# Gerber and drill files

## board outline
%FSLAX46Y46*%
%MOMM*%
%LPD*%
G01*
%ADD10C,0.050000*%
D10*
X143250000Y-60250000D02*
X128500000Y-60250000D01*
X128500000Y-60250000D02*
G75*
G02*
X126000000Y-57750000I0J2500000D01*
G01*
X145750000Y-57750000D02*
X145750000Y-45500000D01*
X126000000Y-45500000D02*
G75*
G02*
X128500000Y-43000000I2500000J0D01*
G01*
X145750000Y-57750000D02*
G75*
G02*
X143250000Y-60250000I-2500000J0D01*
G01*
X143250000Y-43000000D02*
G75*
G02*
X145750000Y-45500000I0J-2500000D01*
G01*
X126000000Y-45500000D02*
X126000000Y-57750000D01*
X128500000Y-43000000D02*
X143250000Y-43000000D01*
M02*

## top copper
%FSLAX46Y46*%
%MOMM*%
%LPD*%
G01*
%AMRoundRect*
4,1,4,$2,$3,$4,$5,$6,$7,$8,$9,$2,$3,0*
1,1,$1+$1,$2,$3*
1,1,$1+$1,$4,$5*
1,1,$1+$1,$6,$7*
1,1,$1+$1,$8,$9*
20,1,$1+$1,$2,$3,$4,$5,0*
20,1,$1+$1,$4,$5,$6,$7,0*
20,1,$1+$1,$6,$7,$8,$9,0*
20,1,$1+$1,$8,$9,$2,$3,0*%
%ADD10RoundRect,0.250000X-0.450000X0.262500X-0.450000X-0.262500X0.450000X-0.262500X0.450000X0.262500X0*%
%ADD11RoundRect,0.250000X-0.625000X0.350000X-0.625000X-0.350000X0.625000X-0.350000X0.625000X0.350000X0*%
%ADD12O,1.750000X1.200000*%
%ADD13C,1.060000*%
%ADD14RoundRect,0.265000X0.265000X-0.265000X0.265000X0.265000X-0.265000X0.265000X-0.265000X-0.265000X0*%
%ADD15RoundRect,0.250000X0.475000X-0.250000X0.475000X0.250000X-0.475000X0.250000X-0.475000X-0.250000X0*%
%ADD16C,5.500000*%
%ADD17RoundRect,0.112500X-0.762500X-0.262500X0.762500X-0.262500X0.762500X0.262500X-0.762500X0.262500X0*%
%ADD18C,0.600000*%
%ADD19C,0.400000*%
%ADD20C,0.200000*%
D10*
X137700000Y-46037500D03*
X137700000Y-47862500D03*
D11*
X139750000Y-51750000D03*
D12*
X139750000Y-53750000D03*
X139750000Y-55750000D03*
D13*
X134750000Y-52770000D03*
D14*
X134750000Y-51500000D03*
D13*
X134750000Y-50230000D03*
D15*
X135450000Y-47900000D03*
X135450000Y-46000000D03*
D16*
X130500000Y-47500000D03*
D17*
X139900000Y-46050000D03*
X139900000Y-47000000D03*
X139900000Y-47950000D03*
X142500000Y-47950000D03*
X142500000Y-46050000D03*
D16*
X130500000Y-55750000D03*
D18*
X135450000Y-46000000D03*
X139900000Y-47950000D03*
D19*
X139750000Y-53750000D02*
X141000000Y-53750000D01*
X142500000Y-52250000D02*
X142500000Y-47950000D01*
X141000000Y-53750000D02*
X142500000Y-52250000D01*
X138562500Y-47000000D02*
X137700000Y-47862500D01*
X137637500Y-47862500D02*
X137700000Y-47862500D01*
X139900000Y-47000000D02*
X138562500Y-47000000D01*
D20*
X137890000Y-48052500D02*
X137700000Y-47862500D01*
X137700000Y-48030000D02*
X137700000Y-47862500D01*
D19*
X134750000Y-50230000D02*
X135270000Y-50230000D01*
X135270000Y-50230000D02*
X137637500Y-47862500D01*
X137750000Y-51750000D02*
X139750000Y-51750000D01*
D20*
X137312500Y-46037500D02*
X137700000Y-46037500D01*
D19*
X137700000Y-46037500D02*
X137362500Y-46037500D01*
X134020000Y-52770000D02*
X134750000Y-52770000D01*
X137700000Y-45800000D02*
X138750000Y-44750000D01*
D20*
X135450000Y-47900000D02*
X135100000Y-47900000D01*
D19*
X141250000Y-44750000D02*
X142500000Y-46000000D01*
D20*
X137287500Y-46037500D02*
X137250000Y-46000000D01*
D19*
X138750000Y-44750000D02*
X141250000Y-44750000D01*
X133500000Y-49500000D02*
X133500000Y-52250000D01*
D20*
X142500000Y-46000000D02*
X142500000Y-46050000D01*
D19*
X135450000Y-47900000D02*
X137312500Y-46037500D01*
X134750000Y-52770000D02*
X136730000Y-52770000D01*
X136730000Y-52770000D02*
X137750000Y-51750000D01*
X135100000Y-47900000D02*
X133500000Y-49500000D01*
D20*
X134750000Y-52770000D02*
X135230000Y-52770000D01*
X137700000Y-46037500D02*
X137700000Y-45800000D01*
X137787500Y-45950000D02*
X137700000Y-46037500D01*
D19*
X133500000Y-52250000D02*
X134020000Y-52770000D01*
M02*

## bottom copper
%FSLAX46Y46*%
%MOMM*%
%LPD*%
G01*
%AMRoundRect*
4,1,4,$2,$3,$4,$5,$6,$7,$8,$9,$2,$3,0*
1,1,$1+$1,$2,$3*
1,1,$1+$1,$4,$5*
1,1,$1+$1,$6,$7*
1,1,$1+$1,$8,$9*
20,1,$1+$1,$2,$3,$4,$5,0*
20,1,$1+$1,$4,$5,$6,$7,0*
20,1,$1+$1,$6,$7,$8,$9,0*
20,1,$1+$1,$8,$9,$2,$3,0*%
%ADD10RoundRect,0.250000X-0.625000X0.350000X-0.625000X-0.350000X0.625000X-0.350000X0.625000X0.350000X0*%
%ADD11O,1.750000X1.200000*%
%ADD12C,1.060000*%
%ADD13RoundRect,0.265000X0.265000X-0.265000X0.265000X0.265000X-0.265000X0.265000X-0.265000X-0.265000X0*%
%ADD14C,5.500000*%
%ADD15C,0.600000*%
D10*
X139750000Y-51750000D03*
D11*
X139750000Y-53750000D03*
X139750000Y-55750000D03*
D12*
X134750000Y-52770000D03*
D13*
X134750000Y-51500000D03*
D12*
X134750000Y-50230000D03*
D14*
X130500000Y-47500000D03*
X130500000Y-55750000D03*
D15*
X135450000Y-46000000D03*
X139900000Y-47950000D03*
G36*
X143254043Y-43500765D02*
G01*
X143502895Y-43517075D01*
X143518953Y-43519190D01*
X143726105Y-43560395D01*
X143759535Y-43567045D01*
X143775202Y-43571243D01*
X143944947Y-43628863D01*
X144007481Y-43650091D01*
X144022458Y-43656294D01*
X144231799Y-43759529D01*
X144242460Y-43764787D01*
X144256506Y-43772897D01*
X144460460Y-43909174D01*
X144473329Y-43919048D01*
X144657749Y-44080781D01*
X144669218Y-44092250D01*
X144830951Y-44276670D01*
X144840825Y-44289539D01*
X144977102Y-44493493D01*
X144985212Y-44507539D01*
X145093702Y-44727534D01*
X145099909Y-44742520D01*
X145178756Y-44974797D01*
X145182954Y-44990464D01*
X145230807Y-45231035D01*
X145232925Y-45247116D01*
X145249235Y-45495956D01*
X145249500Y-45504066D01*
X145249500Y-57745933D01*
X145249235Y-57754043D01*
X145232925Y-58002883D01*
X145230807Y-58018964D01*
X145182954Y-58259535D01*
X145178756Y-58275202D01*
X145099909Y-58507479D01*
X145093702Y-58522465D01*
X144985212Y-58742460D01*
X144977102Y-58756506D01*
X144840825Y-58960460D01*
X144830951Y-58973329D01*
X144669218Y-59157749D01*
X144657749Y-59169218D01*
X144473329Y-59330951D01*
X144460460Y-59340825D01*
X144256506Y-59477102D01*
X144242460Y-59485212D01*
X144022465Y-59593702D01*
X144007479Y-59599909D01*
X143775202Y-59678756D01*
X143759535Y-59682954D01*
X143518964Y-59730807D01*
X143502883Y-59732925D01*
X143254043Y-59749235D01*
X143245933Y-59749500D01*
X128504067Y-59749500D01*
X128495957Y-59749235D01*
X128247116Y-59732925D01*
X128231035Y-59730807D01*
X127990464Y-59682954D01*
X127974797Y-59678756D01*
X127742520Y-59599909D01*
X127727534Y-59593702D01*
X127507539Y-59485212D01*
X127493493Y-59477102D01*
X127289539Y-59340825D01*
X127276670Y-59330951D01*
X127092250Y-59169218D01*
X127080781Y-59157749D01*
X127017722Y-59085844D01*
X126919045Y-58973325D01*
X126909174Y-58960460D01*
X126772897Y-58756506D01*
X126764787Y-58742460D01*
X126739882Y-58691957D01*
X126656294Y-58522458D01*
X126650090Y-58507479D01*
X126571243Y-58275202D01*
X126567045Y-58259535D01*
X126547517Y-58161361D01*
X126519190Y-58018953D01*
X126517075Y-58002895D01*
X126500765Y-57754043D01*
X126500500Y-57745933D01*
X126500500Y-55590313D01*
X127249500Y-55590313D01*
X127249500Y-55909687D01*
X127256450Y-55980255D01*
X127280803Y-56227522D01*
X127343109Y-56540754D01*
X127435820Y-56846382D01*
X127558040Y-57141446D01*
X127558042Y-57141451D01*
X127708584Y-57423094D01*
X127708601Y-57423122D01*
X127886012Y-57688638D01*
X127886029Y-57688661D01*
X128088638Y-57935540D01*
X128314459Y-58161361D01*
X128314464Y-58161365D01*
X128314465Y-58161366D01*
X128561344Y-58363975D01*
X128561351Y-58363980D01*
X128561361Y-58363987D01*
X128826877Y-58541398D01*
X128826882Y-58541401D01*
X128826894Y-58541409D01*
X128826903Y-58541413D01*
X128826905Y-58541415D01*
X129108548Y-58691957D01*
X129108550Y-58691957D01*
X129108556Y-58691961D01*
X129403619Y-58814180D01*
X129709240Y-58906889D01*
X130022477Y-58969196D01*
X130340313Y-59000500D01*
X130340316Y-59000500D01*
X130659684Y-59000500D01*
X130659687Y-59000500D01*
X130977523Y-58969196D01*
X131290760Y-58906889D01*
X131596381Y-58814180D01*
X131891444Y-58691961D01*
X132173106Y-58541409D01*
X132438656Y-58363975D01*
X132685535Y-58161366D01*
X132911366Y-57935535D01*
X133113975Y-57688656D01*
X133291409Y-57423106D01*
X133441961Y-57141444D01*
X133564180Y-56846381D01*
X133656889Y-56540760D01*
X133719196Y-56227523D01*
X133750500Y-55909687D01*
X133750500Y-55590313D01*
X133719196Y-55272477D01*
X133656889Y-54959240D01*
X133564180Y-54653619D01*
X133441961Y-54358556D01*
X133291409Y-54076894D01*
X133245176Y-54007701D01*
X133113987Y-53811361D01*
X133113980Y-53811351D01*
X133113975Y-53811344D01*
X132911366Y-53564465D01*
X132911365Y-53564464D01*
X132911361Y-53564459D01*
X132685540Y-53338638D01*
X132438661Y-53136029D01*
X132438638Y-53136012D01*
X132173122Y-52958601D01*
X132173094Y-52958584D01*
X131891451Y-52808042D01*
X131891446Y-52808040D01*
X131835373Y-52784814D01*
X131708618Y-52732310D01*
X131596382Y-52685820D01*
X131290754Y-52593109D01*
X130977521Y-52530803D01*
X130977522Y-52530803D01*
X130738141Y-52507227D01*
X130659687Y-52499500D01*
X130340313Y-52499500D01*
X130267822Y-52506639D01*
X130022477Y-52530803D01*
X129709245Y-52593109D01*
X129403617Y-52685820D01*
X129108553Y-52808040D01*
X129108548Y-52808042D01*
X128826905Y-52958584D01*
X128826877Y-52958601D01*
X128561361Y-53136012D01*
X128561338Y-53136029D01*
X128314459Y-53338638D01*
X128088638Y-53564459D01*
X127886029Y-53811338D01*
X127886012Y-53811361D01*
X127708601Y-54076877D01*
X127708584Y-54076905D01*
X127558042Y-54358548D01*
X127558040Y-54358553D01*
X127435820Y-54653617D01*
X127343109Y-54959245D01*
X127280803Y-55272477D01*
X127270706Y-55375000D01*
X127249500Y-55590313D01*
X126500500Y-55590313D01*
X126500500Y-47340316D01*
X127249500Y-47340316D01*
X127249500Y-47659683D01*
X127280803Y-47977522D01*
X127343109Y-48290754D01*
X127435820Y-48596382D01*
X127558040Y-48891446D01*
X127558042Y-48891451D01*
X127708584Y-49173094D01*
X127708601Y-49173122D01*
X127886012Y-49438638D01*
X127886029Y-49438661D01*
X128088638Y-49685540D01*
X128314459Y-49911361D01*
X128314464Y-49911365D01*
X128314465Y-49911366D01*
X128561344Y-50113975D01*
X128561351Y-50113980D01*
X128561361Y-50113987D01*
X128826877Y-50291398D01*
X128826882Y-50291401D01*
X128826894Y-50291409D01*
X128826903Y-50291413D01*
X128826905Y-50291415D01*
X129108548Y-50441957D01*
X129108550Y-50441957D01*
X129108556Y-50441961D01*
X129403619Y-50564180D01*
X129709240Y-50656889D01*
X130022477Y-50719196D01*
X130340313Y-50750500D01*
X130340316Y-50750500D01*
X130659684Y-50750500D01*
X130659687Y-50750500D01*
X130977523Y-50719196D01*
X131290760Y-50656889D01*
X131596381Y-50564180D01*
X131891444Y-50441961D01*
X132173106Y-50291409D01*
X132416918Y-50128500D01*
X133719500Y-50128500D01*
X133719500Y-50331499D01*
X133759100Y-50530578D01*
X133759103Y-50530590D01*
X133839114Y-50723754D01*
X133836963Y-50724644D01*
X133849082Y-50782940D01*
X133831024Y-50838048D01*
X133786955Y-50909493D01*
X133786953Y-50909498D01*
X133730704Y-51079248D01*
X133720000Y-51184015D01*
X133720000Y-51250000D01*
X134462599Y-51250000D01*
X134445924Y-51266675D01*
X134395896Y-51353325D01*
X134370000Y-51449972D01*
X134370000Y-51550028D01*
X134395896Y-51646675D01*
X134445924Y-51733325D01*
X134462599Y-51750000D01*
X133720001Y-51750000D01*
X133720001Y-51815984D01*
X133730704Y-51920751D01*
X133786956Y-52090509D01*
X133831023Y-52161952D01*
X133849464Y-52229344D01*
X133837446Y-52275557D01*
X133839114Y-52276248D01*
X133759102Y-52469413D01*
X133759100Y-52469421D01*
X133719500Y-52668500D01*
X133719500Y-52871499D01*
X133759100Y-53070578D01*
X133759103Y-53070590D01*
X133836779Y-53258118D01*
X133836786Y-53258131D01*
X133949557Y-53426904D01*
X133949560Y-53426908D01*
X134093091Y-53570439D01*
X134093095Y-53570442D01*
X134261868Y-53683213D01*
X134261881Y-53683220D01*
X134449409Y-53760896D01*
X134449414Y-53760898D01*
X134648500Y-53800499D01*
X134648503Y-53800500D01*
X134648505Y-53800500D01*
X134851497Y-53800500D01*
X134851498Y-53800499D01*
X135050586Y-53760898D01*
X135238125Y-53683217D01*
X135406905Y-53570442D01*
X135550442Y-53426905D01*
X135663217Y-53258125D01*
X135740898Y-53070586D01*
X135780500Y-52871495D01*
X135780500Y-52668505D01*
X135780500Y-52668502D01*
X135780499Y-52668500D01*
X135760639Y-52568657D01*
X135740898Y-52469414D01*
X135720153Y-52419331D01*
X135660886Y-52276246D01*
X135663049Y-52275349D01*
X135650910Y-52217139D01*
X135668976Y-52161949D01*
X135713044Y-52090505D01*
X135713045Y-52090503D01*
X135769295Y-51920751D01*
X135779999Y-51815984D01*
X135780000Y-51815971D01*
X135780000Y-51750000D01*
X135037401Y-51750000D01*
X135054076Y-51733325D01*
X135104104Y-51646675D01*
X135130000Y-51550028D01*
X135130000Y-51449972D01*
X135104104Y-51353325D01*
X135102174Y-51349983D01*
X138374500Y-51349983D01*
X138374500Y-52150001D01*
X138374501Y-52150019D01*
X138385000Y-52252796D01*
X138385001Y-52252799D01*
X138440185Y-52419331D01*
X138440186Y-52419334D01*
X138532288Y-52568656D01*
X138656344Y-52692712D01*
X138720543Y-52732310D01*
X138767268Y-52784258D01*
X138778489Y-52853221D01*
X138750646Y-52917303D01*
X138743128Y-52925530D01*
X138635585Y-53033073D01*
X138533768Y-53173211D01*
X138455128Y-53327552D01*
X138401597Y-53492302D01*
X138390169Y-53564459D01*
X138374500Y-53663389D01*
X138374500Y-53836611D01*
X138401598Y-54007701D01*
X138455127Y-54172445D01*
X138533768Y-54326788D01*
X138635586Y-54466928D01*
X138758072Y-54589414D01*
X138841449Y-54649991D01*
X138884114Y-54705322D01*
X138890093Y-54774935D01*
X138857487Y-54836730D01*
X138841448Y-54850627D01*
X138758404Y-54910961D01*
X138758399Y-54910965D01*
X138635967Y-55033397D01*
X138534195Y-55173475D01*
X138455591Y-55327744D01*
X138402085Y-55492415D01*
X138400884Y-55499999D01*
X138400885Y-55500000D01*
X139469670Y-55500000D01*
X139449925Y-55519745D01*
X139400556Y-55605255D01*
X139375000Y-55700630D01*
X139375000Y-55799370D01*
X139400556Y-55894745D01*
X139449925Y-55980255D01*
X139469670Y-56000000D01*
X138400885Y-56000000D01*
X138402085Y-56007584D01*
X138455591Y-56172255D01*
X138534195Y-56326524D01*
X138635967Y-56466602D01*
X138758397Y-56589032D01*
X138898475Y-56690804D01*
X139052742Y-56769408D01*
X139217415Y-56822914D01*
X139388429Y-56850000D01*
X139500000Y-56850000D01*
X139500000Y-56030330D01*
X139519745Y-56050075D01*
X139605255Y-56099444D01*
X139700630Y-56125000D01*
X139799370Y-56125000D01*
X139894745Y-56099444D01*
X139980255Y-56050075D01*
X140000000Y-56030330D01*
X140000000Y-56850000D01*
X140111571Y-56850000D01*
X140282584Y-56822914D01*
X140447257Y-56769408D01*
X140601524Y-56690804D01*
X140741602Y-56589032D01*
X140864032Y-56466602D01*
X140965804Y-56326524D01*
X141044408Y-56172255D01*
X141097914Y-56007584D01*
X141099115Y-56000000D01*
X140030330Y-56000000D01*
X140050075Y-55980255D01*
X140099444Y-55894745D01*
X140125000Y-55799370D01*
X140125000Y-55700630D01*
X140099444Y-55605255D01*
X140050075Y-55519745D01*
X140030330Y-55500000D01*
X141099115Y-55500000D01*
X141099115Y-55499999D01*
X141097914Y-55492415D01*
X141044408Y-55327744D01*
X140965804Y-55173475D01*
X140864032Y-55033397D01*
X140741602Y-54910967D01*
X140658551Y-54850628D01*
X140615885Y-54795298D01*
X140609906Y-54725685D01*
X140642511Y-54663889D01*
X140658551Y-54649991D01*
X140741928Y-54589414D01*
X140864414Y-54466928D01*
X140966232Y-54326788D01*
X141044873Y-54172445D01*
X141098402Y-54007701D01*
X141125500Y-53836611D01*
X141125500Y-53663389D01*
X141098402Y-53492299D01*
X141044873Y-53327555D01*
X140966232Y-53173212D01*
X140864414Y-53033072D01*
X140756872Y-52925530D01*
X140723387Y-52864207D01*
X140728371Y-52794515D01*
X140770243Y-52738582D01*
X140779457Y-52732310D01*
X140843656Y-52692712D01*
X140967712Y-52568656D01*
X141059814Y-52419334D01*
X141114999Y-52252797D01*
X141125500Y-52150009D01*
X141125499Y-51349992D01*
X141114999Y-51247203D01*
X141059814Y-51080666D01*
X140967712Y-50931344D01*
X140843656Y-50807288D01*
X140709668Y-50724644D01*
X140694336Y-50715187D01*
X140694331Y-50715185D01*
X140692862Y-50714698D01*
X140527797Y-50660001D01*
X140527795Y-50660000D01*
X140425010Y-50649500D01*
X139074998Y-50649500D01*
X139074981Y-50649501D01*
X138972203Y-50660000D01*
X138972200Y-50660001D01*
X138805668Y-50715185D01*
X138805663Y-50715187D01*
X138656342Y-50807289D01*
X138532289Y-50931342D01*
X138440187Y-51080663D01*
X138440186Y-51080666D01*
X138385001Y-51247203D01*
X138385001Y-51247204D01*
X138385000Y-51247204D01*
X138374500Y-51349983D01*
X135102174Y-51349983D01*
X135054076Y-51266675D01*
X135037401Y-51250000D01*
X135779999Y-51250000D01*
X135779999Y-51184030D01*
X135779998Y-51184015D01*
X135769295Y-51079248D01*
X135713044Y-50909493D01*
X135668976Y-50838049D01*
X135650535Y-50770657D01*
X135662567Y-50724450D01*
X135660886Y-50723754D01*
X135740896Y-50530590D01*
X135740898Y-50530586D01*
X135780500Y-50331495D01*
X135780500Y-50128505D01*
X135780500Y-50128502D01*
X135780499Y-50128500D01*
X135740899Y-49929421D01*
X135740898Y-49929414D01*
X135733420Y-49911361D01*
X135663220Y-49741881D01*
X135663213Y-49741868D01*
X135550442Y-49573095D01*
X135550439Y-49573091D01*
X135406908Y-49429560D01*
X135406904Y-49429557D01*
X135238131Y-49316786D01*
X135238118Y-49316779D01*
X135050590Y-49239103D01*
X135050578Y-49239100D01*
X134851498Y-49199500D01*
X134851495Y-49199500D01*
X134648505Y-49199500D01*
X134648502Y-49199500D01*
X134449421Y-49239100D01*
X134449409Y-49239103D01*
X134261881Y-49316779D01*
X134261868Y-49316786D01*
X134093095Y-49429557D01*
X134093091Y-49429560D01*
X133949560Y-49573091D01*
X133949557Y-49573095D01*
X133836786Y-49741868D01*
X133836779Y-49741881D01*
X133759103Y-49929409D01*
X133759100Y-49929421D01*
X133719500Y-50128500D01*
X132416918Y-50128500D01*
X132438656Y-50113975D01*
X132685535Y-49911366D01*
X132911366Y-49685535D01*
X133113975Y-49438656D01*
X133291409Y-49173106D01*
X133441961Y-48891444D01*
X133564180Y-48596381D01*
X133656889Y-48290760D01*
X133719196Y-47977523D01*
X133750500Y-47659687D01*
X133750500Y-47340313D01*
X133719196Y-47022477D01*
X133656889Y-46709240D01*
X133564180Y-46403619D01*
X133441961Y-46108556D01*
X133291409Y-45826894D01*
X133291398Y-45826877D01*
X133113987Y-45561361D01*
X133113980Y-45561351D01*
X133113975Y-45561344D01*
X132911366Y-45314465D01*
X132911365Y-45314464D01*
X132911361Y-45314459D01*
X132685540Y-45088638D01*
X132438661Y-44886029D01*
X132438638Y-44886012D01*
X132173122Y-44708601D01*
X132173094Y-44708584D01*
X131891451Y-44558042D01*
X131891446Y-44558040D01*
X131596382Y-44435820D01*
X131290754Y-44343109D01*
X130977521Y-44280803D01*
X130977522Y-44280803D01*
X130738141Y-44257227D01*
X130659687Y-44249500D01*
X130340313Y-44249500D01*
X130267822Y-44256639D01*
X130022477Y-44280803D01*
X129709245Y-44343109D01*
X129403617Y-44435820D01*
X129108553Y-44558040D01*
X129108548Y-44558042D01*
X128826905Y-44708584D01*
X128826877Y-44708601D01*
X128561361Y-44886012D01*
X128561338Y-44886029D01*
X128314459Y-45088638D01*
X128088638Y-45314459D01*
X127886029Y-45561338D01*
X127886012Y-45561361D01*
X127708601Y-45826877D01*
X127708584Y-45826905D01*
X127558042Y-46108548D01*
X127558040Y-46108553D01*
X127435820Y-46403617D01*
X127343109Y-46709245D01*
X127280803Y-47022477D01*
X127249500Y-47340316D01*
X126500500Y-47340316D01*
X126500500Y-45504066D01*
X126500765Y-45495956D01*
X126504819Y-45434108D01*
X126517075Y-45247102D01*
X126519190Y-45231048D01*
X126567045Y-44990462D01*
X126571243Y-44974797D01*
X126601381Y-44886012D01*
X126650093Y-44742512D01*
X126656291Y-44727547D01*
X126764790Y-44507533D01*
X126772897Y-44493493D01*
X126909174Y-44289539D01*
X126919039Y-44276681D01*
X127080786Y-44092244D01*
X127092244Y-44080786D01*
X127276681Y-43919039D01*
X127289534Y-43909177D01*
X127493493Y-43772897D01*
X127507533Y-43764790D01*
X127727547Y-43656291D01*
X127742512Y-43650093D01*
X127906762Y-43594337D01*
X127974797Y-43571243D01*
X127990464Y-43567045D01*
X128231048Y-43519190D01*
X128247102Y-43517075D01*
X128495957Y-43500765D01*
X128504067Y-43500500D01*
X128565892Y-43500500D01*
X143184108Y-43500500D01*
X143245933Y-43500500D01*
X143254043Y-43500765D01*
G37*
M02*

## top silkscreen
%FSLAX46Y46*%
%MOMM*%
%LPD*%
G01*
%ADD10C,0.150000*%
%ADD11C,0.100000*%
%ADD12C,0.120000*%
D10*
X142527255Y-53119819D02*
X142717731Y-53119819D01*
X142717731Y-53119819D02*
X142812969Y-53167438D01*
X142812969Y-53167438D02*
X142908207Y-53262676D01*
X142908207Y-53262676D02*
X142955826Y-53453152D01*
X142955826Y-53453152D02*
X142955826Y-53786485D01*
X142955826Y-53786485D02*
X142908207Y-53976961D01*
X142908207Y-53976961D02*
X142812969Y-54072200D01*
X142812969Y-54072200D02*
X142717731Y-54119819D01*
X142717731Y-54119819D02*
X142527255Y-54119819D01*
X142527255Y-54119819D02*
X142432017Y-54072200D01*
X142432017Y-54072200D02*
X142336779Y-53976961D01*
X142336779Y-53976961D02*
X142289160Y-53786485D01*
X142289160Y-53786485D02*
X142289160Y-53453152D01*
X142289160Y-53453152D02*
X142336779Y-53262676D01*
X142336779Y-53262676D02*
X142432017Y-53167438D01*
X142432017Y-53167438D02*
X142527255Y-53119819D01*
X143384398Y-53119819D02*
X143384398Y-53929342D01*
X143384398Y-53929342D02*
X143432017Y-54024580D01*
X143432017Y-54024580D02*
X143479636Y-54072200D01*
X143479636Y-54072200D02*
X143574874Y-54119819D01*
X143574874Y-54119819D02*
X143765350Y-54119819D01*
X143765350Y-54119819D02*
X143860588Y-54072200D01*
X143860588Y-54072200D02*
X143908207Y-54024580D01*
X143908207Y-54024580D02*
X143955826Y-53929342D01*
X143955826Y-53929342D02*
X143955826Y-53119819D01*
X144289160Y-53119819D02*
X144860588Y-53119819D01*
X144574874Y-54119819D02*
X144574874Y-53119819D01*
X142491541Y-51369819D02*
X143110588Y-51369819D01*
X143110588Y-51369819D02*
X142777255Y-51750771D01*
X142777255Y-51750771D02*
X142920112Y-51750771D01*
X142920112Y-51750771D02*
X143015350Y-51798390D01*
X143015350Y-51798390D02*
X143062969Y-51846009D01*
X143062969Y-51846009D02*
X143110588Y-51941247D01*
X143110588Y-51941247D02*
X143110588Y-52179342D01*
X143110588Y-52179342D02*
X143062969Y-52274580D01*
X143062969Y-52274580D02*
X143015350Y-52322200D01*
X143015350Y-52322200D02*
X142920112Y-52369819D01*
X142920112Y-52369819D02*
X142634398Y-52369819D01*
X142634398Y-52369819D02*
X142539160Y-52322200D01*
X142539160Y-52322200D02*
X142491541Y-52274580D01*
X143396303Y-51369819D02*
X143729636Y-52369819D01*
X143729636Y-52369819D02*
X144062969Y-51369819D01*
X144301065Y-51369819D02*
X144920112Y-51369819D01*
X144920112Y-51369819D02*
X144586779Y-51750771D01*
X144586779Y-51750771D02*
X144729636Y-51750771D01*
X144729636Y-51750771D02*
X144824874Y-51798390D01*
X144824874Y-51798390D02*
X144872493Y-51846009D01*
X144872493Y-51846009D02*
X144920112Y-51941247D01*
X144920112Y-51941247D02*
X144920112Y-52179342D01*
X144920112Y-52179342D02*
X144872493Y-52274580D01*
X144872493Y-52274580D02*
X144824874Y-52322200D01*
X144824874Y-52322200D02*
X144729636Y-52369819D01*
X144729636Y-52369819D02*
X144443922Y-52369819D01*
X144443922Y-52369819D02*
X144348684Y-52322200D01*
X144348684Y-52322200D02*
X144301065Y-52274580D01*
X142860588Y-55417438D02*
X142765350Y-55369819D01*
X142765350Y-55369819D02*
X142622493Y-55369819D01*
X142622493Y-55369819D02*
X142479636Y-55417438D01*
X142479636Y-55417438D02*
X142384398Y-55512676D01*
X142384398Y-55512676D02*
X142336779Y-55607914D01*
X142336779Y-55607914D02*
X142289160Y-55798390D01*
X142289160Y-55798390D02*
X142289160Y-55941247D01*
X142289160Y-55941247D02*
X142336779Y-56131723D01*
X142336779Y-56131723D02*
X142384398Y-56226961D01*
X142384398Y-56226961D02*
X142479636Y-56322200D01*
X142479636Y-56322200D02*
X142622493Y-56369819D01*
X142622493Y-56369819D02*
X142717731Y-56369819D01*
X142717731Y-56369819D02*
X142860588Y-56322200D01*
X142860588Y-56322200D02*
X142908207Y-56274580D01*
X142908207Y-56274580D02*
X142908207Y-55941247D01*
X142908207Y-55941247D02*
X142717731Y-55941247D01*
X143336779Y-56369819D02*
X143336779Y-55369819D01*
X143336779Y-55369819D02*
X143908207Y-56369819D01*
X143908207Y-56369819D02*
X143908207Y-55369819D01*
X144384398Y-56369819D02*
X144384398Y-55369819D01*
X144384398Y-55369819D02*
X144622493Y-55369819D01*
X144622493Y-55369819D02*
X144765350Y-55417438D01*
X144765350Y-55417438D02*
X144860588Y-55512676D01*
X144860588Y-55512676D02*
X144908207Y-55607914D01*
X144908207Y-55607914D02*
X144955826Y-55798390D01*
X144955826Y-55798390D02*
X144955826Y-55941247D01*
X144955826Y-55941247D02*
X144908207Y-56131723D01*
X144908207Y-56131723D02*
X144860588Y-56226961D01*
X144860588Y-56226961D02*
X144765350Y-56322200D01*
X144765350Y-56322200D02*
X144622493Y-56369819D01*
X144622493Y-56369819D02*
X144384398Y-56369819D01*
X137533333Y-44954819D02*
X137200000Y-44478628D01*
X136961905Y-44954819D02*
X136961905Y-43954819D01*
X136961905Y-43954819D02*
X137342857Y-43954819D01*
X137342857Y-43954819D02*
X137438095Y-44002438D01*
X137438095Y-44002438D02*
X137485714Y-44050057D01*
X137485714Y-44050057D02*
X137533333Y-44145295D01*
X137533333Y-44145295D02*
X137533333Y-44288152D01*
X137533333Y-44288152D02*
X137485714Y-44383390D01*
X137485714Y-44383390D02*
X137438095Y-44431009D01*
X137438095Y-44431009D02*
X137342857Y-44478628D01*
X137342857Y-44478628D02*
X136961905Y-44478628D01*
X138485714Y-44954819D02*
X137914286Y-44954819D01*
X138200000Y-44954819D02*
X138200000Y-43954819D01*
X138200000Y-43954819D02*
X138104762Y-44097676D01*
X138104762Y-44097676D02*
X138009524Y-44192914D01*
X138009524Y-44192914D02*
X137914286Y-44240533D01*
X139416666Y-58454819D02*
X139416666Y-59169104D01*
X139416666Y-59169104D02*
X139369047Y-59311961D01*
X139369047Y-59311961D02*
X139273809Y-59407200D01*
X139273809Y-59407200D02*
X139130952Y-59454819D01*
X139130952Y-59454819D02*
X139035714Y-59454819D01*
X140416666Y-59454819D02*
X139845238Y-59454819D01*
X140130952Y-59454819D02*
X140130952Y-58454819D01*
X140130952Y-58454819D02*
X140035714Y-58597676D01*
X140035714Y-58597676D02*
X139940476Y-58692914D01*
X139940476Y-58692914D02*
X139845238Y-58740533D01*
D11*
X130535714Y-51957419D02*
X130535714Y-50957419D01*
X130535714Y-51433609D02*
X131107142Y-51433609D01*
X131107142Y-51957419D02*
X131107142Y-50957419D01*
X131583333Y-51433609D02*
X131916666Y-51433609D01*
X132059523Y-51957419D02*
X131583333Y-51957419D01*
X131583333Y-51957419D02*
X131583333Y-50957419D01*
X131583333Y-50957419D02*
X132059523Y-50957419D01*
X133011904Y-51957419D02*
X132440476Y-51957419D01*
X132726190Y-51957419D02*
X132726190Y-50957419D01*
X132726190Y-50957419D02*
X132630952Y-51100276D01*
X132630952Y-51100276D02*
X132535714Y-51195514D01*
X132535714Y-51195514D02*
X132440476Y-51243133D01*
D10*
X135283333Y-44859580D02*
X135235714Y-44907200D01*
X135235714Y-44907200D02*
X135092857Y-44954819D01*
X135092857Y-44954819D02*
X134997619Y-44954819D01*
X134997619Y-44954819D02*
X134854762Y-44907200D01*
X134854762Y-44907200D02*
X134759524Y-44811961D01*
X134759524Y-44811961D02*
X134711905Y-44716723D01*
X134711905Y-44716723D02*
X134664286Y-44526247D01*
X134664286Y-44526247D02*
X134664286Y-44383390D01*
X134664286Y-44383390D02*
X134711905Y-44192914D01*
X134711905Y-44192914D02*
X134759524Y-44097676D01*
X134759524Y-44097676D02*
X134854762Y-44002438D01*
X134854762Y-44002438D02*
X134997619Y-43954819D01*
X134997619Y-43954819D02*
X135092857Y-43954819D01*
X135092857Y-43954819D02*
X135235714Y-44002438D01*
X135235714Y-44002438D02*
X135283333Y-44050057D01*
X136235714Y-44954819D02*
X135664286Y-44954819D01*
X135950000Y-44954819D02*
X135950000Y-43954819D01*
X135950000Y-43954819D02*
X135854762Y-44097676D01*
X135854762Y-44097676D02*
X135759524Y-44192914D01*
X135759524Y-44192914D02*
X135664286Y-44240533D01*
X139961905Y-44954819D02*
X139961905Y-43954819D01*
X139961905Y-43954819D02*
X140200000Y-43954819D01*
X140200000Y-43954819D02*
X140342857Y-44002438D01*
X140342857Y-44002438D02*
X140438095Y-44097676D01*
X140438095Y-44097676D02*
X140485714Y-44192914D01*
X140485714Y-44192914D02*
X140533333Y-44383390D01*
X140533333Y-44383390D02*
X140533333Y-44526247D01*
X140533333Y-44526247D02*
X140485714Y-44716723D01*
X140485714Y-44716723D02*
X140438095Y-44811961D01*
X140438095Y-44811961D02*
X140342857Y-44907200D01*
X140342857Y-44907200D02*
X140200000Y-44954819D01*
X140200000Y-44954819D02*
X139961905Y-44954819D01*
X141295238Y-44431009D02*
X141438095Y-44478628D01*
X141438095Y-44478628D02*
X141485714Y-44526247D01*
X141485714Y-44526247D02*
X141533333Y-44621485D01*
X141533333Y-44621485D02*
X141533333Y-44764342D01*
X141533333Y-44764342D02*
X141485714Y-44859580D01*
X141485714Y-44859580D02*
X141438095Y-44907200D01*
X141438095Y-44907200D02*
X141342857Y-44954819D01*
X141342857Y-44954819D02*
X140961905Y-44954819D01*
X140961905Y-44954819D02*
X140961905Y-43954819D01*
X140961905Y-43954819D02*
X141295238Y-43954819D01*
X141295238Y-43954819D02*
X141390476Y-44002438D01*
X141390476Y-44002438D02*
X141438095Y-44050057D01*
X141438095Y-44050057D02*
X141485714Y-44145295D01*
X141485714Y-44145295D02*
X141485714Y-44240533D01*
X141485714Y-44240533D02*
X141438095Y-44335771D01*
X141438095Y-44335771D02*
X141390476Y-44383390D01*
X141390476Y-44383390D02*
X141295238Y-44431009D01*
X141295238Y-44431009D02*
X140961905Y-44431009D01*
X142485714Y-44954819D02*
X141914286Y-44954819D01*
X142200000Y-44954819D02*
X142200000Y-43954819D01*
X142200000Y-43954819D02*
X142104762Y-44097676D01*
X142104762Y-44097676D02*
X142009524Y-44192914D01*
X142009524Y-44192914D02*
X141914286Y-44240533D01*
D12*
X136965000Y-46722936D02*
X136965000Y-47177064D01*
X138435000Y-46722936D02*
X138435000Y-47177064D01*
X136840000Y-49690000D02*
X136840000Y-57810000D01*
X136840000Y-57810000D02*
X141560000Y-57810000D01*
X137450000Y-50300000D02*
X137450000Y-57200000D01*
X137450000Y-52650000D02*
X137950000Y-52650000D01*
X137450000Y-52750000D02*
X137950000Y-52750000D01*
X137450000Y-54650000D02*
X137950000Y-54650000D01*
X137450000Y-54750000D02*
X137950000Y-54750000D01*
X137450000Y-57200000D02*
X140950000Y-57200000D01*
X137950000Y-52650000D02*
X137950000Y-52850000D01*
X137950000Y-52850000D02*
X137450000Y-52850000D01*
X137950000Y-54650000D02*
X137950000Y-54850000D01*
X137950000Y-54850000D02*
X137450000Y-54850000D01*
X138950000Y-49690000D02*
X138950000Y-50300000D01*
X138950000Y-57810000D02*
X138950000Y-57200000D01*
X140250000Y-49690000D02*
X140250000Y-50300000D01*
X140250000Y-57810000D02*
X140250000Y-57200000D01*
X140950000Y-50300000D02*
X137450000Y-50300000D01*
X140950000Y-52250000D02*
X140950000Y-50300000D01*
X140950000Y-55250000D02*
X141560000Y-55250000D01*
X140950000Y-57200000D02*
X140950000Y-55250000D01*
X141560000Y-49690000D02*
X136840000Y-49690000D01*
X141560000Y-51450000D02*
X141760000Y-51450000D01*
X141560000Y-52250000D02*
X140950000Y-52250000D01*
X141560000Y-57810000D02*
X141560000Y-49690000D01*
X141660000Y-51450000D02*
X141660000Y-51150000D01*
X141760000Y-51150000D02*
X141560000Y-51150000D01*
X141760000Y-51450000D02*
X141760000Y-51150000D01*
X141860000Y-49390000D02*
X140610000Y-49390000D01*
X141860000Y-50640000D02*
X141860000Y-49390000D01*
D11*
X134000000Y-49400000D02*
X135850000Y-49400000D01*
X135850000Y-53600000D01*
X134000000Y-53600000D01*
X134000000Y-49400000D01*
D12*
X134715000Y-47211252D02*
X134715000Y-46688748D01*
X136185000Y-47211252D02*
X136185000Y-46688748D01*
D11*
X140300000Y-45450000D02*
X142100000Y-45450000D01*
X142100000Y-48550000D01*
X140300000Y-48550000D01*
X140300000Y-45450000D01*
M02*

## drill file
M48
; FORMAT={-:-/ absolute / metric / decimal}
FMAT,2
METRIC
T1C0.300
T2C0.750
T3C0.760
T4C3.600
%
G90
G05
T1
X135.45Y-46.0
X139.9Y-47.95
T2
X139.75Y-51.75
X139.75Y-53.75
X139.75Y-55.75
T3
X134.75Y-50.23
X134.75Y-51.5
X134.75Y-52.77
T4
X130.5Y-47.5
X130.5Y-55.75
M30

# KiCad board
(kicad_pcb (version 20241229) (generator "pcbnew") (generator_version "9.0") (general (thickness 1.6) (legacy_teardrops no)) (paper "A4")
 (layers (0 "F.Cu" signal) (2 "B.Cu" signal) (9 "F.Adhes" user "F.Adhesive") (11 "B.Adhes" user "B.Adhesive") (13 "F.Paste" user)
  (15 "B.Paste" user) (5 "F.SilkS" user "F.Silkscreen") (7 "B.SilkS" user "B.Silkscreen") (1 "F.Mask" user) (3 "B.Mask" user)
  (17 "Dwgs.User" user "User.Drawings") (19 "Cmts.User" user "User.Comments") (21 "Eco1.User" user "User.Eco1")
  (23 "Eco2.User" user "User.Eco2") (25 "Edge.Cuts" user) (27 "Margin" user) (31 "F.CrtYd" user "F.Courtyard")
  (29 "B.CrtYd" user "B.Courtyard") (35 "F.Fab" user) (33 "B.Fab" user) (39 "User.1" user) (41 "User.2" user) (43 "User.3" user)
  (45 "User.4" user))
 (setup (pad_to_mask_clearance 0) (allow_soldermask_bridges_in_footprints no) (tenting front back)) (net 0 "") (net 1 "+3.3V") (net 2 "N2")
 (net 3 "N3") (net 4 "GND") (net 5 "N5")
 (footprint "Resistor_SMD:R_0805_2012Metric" (layer "F.Cu") (at 137.7 46.95 -90)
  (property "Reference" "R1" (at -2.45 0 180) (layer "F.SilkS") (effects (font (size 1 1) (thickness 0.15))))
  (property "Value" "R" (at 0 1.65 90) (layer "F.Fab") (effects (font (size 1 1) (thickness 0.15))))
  (fp_line (start -0.227064 0.735) (end 0.227064 0.735) (stroke (width 0.12) (type solid)) (layer "F.SilkS"))
  (fp_line (start -0.227064 -0.735) (end 0.227064 -0.735) (stroke (width 0.12) (type solid)) (layer "F.SilkS"))
  (pad "1" smd roundrect (at -0.9125 0 270) (size 1.025 1.4) (layers "F.Cu" "F.Mask" "F.Paste") (roundrect_rratio 0.243902) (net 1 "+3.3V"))
  (pad "2" smd roundrect (at 0.9125 0 270) (size 1.025 1.4) (layers "F.Cu" "F.Mask" "F.Paste") (roundrect_rratio 0.243902) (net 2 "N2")))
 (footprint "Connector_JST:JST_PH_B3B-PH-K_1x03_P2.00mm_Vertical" (layer "F.Cu") (at 139.75 51.75 -90)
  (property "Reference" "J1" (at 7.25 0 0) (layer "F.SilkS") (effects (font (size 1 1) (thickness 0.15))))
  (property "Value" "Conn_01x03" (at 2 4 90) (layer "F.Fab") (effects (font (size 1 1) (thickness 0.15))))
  (fp_line (start -2.06 2.91) (end 6.06 2.91) (stroke (width 0.12) (type solid)) (layer "F.SilkS"))
  (fp_line (start 6.06 2.91) (end 6.06 -1.81) (stroke (width 0.12) (type solid)) (layer "F.SilkS"))
  (fp_line (start -1.45 2.3) (end 5.45 2.3) (stroke (width 0.12) (type solid)) (layer "F.SilkS"))
  (fp_line (start 0.9 2.3) (end 0.9 1.8) (stroke (width 0.12) (type solid)) (layer "F.SilkS"))
  (fp_line (start 1 2.3) (end 1 1.8) (stroke (width 0.12) (type solid)) (layer "F.SilkS"))
  (fp_line (start 2.9 2.3) (end 2.9 1.8) (stroke (width 0.12) (type solid)) (layer "F.SilkS"))
  (fp_line (start 3 2.3) (end 3 1.8) (stroke (width 0.12) (type solid)) (layer "F.SilkS"))
  (fp_line (start 5.45 2.3) (end 5.45 -1.2) (stroke (width 0.12) (type solid)) (layer "F.SilkS"))
  (fp_line (start 0.9 1.8) (end 1.1 1.8) (stroke (width 0.12) (type solid)) (layer "F.SilkS"))
  (fp_line (start 1.1 1.8) (end 1.1 2.3) (stroke (width 0.12) (type solid)) (layer "F.SilkS"))
  (fp_line (start 2.9 1.8) (end 3.1 1.8) (stroke (width 0.12) (type solid)) (layer "F.SilkS"))
  (fp_line (start 3.1 1.8) (end 3.1 2.3) (stroke (width 0.12) (type solid)) (layer "F.SilkS"))
  (fp_line (start -2.06 0.8) (end -1.45 0.8) (stroke (width 0.12) (type solid)) (layer "F.SilkS"))
  (fp_line (start 6.06 0.8) (end 5.45 0.8) (stroke (width 0.12) (type solid)) (layer "F.SilkS"))
  (fp_line (start -2.06 -0.5) (end -1.45 -0.5) (stroke (width 0.12) (type solid)) (layer "F.SilkS"))
  (fp_line (start 6.06 -0.5) (end 5.45 -0.5) (stroke (width 0.12) (type solid)) (layer "F.SilkS"))
  (fp_line (start -1.45 -1.2) (end -1.45 2.3) (stroke (width 0.12) (type solid)) (layer "F.SilkS"))
  (fp_line (start 0.5 -1.2) (end -1.45 -1.2) (stroke (width 0.12) (type solid)) (layer "F.SilkS"))
  (fp_line (start 3.5 -1.2) (end 3.5 -1.81) (stroke (width 0.12) (type solid)) (layer "F.SilkS"))
  (fp_line (start 5.45 -1.2) (end 3.5 -1.2) (stroke (width 0.12) (type solid)) (layer "F.SilkS"))
  (fp_line (start -2.06 -1.81) (end -2.06 2.91) (stroke (width 0.12) (type solid)) (layer "F.SilkS"))
  (fp_line (start -0.3 -1.81) (end -0.3 -2.01) (stroke (width 0.12) (type solid)) (layer "F.SilkS"))
  (fp_line (start 0.5 -1.81) (end 0.5 -1.2) (stroke (width 0.12) (type solid)) (layer "F.SilkS"))
  (fp_line (start 6.06 -1.81) (end -2.06 -1.81) (stroke (width 0.12) (type solid)) (layer "F.SilkS"))
  (fp_line (start -0.3 -1.91) (end -0.6 -1.91) (stroke (width 0.12) (type solid)) (layer "F.SilkS"))
  (fp_line (start -0.6 -2.01) (end -0.6 -1.81) (stroke (width 0.12) (type solid)) (layer "F.SilkS"))
  (fp_line (start -0.3 -2.01) (end -0.6 -2.01) (stroke (width 0.12) (type solid)) (layer "F.SilkS"))
  (fp_line (start -2.36 -2.11) (end -2.36 -0.86) (stroke (width 0.12) (type solid)) (layer "F.SilkS"))
  (fp_line (start -1.11 -2.11) (end -2.36 -2.11) (stroke (width 0.12) (type solid)) (layer "F.SilkS"))
  (pad "1" thru_hole roundrect (at 0 0 270) (size 1.2 1.75) (drill 0.75) (layers "*.Cu" "*.Mask") (remove_unused_layers no)
   (roundrect_rratio 0.208333) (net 1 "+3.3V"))
  (pad "2" thru_hole oval (at 2 0 270) (size 1.2 1.75) (drill 0.75) (layers "*.Cu" "*.Mask") (remove_unused_layers no) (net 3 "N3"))
  (pad "3" thru_hole oval (at 4 0 270) (size 1.2 1.75) (drill 0.75) (layers "*.Cu" "*.Mask") (remove_unused_layers no) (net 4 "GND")))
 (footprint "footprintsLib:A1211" (layer "F.Cu") (at 134.75 51.5 90)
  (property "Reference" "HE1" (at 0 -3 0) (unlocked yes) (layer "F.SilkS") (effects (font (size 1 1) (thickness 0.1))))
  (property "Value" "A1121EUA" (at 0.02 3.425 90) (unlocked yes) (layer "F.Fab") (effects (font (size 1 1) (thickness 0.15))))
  (fp_rect (start -2.1 -0.75) (end 2.1 1.1) (stroke (width 0.1) (type solid)) (fill no) (layer "F.SilkS"))
  (pad "1" thru_hole circle (at -1.27 0 90) (size 1.06 1.06) (drill 0.76) (layers "*.Cu" "*.Mask") (remove_unused_layers no) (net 1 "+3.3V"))
  (pad "2" thru_hole roundrect (at 0 0 90) (size 1.06 1.06) (drill 0.76) (layers "*.Cu" "*.Mask") (remove_unused_layers no)
   (roundrect_rratio 0.25) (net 4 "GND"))
  (pad "3" thru_hole circle (at 1.27 0 90) (size 1.06 1.06) (drill 0.76) (layers "*.Cu" "*.Mask") (remove_unused_layers no) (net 2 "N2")))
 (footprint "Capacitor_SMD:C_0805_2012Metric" (layer "F.Cu") (at 135.45 46.95 90)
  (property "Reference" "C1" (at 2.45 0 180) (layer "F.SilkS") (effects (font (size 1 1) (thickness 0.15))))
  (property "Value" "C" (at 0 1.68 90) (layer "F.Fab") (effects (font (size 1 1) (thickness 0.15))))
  (fp_line (start -0.261252 -0.735) (end 0.261252 -0.735) (stroke (width 0.12) (type solid)) (layer "F.SilkS"))
  (fp_line (start -0.261252 0.735) (end 0.261252 0.735) (stroke (width 0.12) (type solid)) (layer "F.SilkS"))
  (pad "1" smd roundrect (at -0.95 0 90) (size 1 1.45) (layers "F.Cu" "F.Mask" "F.Paste") (roundrect_rratio 0.25) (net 1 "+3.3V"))
  (pad "2" smd roundrect (at 0.95 0 90) (size 1 1.45) (layers "F.Cu" "F.Mask" "F.Paste") (roundrect_rratio 0.25) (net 4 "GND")))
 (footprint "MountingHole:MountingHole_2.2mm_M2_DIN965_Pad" (layer "F.Cu") (at 130.5 47.5)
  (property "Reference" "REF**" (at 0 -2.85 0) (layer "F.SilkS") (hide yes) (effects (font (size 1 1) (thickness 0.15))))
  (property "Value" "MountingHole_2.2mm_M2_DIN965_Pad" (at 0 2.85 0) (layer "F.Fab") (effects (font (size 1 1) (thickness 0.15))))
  (pad "1" thru_hole circle (at 0 0) (size 5.5 5.5) (drill 3.6) (layers "*.Cu" "*.Mask") (remove_unused_layers no) (zone_connect 2)))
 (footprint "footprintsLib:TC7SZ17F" (layer "F.Cu") (at 141.2 47 -90)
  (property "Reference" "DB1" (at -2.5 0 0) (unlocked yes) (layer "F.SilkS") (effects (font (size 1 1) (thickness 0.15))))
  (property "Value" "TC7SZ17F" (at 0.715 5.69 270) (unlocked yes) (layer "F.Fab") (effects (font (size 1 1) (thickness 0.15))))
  (fp_rect (start -1.55 -0.9) (end 1.55 0.9) (stroke (width 0.1) (type solid)) (fill no) (layer "F.SilkS"))
  (pad "1" smd roundrect (at -0.95 1.3) (size 1.75 0.75) (layers "F.Cu" "F.Mask" "F.Paste") (roundrect_rratio 0.15) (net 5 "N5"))
  (pad "2" smd roundrect (at 0 1.3) (size 1.75 0.75) (layers "F.Cu" "F.Mask" "F.Paste") (roundrect_rratio 0.15) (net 2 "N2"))
  (pad "3" smd roundrect (at 0.95 1.3) (size 1.75 0.75) (layers "F.Cu" "F.Mask" "F.Paste") (roundrect_rratio 0.15) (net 4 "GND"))
  (pad "4" smd roundrect (at 0.95 -1.3) (size 1.75 0.75) (layers "F.Cu" "F.Mask" "F.Paste") (roundrect_rratio 0.15) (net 3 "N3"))
  (pad "5" smd roundrect (at -0.95 -1.3) (size 1.75 0.75) (layers "F.Cu" "F.Mask" "F.Paste") (roundrect_rratio 0.15) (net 1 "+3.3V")))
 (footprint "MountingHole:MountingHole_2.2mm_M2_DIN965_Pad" (layer "F.Cu") (at 130.5 55.75)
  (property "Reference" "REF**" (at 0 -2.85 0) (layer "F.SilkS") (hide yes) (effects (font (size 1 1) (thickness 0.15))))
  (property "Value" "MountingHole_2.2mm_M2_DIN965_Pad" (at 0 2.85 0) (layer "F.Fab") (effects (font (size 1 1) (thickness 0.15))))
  (pad "1" thru_hole circle (at 0 0) (size 5.5 5.5) (drill 3.6) (layers "*.Cu" "*.Mask") (remove_unused_layers no) (zone_connect 2)))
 (gr_line (start 143.25 60.25) (end 128.5 60.25) (stroke (width 0.05) (type default)) (layer "Edge.Cuts"))
 (gr_arc (start 128.5 60.25) (mid 126.732233 59.517767) (end 126 57.75) (stroke (width 0.05) (type default)) (layer "Edge.Cuts"))
 (gr_line (start 145.75 57.75) (end 145.75 45.5) (stroke (width 0.05) (type default)) (layer "Edge.Cuts"))
 (gr_arc (start 126 45.5) (mid 126.732233 43.732233) (end 128.5 43) (stroke (width 0.05) (type default)) (layer "Edge.Cuts"))
 (gr_arc (start 145.75 57.75) (mid 145.017767 59.517767) (end 143.25 60.25) (stroke (width 0.05) (type default)) (layer "Edge.Cuts"))
 (gr_arc (start 143.25 43) (mid 145.017767 43.732233) (end 145.75 45.5) (stroke (width 0.05) (type default)) (layer "Edge.Cuts"))
 (gr_line (start 126 45.5) (end 126 57.75) (stroke (width 0.05) (type default)) (layer "Edge.Cuts"))
 (gr_line (start 128.5 43) (end 143.25 43) (stroke (width 0.05) (type default)) (layer "Edge.Cuts"))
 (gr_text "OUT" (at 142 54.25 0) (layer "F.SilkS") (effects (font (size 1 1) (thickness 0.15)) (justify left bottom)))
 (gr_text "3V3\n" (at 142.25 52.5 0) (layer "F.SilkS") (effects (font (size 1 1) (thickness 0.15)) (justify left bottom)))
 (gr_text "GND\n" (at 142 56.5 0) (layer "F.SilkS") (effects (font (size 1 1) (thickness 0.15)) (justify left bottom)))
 (via (at 135.45 46) (size 0.6) (drill 0.3) (layers "F.Cu" "B.Cu") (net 4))
 (via (at 139.9 47.95) (size 0.6) (drill 0.3) (layers "F.Cu" "B.Cu") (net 4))
 (segment (start 139.75 53.75) (end 141 53.75) (width 0.4) (layer "F.Cu") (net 3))
 (segment (start 142.5 52.25) (end 142.5 47.95) (width 0.4) (layer "F.Cu") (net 3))
 (segment (start 141 53.75) (end 142.5 52.25) (width 0.4) (layer "F.Cu") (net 3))
 (segment (start 138.5625 47) (end 137.7 47.8625) (width 0.4) (layer "F.Cu") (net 2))
 (segment (start 137.6375 47.8625) (end 137.7 47.8625) (width 0.4) (layer "F.Cu") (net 2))
 (segment (start 139.9 47) (end 138.5625 47) (width 0.4) (layer "F.Cu") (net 2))
 (segment (start 137.89 48.0525) (end 137.7 47.8625) (width 0.2) (layer "F.Cu") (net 2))
 (segment (start 137.7 48.03) (end 137.7 47.8625) (width 0.2) (layer "F.Cu") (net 2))
 (segment (start 134.75 50.23) (end 135.27 50.23) (width 0.4) (layer "F.Cu") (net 2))
 (segment (start 135.27 50.23) (end 137.6375 47.8625) (width 0.4) (layer "F.Cu") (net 2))
 (segment (start 137.75 51.75) (end 139.75 51.75) (width 0.4) (layer "F.Cu") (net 1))
 (segment (start 137.3125 46.0375) (end 137.7 46.0375) (width 0.2) (layer "F.Cu") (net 1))
 (segment (start 137.7 46.0375) (end 137.3625 46.0375) (width 0.4) (layer "F.Cu") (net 1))
 (segment (start 134.02 52.77) (end 134.75 52.77) (width 0.4) (layer "F.Cu") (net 1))
 (segment (start 137.7 45.8) (end 138.75 44.75) (width 0.4) (layer "F.Cu") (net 1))
 (segment (start 135.45 47.9) (end 135.1 47.9) (width 0.2) (layer "F.Cu") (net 1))
 (segment (start 141.25 44.75) (end 142.5 46) (width 0.4) (layer "F.Cu") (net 1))
 (segment (start 137.2875 46.0375) (end 137.25 46) (width 0.2) (layer "F.Cu") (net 1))
 (segment (start 138.75 44.75) (end 141.25 44.75) (width 0.4) (layer "F.Cu") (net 1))
 (segment (start 133.5 49.5) (end 133.5 52.25) (width 0.4) (layer "F.Cu") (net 1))
 (segment (start 142.5 46) (end 142.5 46.05) (width 0.2) (layer "F.Cu") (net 1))
 (segment (start 135.45 47.9) (end 137.3125 46.0375) (width 0.4) (layer "F.Cu") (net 1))
 (segment (start 134.75 52.77) (end 136.73 52.77) (width 0.4) (layer "F.Cu") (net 1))
 (segment (start 136.73 52.77) (end 137.75 51.75) (width 0.4) (layer "F.Cu") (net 1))
 (segment (start 135.1 47.9) (end 133.5 49.5) (width 0.4) (layer "F.Cu") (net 1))
 (segment (start 134.75 52.77) (end 135.23 52.77) (width 0.2) (layer "F.Cu") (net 1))
 (segment (start 137.7 46.0375) (end 137.7 45.8) (width 0.2) (layer "F.Cu") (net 1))
 (segment (start 137.7875 45.95) (end 137.7 46.0375) (width 0.2) (layer "F.Cu") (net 1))
 (segment (start 133.5 52.25) (end 134.02 52.77) (width 0.4) (layer "F.Cu") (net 1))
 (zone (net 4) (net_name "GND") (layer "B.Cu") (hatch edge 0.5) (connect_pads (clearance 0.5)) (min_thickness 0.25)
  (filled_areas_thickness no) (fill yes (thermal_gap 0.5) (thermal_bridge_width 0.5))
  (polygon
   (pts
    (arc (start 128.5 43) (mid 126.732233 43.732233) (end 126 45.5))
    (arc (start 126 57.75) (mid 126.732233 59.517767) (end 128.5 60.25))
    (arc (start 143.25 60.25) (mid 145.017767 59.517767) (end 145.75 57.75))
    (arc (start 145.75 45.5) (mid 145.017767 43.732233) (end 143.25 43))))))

